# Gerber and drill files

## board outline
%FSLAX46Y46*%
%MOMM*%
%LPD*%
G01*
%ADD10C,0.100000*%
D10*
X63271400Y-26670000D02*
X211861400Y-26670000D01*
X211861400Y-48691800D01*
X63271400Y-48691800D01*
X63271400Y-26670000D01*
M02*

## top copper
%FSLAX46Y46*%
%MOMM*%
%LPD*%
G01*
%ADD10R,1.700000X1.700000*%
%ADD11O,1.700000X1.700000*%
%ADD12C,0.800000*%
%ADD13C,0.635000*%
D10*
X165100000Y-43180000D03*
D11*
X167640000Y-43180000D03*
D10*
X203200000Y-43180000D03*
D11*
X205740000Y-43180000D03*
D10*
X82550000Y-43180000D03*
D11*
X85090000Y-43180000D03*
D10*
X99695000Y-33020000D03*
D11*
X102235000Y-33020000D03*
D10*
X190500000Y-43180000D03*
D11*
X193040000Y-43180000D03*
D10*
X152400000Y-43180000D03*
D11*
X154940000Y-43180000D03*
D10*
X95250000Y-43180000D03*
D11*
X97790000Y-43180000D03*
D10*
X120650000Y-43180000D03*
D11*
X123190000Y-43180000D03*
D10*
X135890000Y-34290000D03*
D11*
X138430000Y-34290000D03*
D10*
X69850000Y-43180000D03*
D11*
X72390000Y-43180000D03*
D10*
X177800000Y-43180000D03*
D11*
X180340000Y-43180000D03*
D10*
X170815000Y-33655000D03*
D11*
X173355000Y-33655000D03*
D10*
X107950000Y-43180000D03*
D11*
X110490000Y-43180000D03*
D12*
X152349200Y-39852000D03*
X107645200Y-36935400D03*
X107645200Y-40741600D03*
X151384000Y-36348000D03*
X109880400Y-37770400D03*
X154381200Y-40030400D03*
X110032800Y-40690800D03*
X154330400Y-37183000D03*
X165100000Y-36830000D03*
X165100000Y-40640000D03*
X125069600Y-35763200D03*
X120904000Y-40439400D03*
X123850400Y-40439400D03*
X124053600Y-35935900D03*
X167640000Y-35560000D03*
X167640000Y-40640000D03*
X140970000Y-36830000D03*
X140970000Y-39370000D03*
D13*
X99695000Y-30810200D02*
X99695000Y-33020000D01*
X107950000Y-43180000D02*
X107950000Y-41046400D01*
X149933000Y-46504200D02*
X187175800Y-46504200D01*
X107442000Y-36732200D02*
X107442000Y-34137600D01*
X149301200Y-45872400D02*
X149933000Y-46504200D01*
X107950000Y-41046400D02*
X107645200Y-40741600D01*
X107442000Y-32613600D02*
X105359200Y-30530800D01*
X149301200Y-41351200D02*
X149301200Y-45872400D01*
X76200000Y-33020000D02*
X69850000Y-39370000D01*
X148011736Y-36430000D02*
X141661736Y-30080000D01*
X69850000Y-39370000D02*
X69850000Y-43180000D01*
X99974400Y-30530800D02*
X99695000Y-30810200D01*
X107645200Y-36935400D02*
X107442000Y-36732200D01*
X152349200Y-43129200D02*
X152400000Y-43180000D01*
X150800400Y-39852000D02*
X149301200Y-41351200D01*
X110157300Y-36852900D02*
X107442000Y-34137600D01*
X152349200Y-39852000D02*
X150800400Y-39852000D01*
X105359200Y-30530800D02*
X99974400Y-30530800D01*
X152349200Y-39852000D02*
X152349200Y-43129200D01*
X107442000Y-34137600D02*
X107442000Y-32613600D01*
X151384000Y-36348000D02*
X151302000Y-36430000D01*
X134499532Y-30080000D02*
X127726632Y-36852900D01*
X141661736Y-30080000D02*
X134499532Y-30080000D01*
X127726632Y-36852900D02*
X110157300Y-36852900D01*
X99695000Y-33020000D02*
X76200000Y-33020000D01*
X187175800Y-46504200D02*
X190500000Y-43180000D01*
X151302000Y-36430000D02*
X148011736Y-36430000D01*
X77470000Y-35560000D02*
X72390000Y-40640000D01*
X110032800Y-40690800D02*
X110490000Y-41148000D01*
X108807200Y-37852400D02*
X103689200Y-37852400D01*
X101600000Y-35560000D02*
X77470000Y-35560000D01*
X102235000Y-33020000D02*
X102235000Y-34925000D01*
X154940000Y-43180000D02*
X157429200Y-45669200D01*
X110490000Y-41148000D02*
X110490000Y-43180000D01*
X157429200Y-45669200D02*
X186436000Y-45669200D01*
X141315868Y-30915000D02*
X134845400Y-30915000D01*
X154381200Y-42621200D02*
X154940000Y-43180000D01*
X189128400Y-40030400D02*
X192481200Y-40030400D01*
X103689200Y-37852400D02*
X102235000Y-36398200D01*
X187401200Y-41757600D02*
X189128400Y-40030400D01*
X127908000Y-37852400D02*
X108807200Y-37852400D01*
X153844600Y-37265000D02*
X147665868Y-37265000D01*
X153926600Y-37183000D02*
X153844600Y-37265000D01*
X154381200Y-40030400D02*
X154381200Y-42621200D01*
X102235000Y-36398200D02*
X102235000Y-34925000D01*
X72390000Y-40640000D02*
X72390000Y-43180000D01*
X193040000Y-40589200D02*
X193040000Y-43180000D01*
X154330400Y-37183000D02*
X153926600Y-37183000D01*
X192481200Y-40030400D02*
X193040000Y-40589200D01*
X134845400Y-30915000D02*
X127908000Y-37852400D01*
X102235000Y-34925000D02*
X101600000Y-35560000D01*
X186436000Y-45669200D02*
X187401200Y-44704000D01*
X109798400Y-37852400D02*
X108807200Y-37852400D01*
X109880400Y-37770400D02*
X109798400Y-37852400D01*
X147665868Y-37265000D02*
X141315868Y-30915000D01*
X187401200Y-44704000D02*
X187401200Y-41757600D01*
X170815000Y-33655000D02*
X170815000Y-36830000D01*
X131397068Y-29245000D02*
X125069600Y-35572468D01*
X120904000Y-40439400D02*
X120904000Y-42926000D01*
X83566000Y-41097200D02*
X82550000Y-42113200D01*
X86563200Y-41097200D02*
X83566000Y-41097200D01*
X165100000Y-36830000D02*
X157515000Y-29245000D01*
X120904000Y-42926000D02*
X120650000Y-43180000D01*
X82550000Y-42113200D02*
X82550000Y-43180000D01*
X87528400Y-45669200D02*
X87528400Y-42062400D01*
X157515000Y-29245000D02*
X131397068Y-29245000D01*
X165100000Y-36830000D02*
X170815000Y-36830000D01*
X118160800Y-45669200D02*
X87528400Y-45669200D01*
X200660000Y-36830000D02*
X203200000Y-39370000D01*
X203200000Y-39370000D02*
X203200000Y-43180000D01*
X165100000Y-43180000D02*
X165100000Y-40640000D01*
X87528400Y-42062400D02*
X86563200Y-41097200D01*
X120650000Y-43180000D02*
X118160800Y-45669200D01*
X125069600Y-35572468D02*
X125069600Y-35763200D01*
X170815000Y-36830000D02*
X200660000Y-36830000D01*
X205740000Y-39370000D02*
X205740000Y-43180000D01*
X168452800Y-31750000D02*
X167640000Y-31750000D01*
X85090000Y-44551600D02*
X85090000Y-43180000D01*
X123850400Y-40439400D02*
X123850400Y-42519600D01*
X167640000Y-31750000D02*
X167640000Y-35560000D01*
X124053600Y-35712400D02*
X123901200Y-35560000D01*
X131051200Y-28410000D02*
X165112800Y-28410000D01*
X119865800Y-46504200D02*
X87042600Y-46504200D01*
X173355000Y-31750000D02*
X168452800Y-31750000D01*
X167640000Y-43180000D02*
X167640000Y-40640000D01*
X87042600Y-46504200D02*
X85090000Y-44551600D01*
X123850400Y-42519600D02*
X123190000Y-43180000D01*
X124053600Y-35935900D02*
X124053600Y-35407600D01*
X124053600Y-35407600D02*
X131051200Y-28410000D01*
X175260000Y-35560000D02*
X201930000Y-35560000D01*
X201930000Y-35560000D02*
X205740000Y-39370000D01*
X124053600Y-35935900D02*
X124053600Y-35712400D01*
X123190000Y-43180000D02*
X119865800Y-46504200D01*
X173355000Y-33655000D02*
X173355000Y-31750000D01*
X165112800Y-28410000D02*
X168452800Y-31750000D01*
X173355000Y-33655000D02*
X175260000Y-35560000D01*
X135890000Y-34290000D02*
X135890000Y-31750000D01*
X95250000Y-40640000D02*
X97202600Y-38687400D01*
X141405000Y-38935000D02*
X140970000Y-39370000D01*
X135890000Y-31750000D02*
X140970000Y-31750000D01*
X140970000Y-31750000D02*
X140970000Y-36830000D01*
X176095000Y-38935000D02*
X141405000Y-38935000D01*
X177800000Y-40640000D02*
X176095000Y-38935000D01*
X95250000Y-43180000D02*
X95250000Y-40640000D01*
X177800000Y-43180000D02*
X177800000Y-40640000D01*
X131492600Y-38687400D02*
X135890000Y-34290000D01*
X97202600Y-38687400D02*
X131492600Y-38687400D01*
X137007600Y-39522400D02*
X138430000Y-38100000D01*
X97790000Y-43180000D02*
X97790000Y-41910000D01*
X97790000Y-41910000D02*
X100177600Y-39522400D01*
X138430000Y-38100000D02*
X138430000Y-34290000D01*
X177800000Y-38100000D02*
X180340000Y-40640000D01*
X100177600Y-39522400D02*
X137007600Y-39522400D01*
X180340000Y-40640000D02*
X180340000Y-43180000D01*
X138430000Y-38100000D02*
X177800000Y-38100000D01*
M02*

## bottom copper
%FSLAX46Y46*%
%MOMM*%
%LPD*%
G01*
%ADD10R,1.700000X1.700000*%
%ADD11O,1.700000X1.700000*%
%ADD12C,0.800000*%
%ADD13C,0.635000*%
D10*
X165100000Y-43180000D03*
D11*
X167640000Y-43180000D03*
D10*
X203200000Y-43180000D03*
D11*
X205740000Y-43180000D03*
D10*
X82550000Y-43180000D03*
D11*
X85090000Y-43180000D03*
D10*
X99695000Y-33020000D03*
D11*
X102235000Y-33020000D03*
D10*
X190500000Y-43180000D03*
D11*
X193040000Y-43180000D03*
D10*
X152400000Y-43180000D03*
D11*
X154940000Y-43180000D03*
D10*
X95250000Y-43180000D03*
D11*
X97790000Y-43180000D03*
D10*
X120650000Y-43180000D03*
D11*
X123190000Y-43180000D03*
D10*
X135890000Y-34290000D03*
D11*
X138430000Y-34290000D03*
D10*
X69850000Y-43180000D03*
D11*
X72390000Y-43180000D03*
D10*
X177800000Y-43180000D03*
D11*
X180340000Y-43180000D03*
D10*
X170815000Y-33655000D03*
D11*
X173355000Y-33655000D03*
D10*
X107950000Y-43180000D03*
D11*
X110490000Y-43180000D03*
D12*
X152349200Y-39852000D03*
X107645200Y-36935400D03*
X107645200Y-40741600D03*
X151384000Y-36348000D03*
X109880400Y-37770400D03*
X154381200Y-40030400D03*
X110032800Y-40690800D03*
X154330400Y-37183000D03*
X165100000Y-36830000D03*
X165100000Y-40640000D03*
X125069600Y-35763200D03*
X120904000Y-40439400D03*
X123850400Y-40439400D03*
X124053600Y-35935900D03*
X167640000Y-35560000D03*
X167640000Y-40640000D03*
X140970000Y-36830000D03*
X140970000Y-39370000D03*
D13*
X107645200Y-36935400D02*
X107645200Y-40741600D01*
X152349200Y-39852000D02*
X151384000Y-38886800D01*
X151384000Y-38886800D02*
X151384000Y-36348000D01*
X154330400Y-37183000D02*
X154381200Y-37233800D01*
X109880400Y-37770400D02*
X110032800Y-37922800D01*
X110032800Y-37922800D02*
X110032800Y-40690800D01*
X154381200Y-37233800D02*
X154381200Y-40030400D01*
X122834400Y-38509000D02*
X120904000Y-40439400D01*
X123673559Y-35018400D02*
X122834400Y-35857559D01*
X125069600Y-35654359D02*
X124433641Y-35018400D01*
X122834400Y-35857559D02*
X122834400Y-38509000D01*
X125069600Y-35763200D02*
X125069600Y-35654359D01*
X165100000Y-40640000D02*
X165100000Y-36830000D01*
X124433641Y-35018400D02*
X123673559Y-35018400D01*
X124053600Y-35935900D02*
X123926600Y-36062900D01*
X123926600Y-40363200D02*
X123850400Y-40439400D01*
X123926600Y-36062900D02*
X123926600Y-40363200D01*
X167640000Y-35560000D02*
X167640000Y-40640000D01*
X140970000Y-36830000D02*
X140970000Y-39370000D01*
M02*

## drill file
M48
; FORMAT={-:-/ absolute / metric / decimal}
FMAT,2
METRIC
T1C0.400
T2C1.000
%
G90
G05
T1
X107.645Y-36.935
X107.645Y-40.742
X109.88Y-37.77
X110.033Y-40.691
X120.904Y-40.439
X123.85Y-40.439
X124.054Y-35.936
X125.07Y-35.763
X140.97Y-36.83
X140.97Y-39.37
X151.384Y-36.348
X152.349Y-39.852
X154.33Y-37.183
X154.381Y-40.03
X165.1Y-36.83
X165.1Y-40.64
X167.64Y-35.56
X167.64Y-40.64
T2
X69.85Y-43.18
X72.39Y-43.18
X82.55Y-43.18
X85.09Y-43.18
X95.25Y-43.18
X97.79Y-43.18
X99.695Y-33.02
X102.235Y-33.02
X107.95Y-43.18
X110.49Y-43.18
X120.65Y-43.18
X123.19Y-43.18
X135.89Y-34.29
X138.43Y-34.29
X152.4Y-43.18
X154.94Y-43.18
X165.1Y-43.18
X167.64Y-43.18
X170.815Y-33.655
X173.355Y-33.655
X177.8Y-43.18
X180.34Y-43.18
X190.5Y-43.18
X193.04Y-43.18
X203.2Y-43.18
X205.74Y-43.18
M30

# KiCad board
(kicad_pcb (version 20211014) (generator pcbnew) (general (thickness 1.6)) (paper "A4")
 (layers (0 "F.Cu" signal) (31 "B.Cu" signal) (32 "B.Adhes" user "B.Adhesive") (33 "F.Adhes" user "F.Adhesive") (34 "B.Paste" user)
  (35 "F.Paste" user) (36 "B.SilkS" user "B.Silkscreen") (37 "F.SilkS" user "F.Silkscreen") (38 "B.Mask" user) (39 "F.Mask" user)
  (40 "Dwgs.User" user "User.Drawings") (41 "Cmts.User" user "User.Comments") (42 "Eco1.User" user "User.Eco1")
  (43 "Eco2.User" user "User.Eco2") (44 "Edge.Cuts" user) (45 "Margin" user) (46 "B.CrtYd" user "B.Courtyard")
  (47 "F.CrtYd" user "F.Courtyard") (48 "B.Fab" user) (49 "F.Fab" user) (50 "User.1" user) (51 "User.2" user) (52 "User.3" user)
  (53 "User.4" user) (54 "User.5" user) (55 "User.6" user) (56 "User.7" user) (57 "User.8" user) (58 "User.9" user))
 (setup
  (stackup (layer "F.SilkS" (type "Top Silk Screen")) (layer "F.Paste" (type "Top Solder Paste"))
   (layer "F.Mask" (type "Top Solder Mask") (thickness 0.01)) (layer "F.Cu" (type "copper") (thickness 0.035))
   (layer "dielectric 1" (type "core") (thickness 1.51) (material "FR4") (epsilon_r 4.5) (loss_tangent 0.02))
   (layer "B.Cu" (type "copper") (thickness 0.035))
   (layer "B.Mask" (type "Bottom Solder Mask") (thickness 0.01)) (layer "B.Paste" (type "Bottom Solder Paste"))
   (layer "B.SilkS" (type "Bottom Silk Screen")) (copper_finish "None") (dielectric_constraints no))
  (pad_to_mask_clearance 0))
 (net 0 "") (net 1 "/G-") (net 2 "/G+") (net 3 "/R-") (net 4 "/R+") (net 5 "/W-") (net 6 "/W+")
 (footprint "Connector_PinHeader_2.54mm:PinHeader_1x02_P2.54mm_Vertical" (layer "F.Cu") (at 165.1 43.18 90)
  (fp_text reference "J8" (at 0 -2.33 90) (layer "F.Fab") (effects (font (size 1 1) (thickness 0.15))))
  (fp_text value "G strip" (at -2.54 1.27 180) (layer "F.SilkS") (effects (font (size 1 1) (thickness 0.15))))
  (pad "1" thru_hole rect (at 0 0 90) (size 1.7 1.7) (drill 1) (layers *.Cu *.Mask) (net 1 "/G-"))
  (pad "2" thru_hole oval (at 0 2.54 90) (size 1.7 1.7) (drill 1) (layers *.Cu *.Mask) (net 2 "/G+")))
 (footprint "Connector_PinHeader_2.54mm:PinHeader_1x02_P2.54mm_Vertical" (layer "F.Cu") (at 203.2 43.18 90)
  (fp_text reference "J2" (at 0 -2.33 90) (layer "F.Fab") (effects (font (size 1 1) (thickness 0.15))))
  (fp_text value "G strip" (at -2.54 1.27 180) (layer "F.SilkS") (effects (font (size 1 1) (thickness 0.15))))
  (pad "1" thru_hole rect (at 0 0 90) (size 1.7 1.7) (drill 1) (layers *.Cu *.Mask) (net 1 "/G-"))
  (pad "2" thru_hole oval (at 0 2.54 90) (size 1.7 1.7) (drill 1) (layers *.Cu *.Mask) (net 2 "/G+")))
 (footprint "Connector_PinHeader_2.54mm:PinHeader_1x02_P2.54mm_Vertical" (layer "F.Cu") (at 82.55 43.18 90)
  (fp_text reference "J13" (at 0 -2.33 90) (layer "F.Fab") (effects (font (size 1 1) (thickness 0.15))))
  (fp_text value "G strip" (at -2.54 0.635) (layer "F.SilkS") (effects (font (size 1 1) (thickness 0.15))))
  (pad "1" thru_hole rect (at 0 0 90) (size 1.7 1.7) (drill 1) (layers *.Cu *.Mask) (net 1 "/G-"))
  (pad "2" thru_hole oval (at 0 2.54 90) (size 1.7 1.7) (drill 1) (layers *.Cu *.Mask) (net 2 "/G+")))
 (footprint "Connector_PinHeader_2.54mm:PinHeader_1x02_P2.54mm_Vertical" (layer "F.Cu") (at 99.695 33.02 90)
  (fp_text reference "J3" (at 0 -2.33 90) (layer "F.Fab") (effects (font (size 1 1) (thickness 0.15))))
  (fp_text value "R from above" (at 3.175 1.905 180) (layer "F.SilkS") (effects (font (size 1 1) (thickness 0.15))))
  (pad "1" thru_hole rect (at 0 0 90) (size 1.7 1.7) (drill 1) (layers *.Cu *.Mask) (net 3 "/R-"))
  (pad "2" thru_hole oval (at 0 2.54 90) (size 1.7 1.7) (drill 1) (layers *.Cu *.Mask) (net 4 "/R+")))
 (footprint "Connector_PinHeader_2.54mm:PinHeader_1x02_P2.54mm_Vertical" (layer "F.Cu") (at 190.5 43.18 90)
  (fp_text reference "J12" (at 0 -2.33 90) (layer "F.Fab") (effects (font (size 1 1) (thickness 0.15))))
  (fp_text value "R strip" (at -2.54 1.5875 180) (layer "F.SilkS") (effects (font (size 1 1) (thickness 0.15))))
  (pad "1" thru_hole rect (at 0 0 90) (size 1.7 1.7) (drill 1) (layers *.Cu *.Mask) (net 3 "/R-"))
  (pad "2" thru_hole oval (at 0 2.54 90) (size 1.7 1.7) (drill 1) (layers *.Cu *.Mask) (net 4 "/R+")))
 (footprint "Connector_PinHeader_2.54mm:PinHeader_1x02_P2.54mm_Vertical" (layer "F.Cu") (at 152.4 43.18 90)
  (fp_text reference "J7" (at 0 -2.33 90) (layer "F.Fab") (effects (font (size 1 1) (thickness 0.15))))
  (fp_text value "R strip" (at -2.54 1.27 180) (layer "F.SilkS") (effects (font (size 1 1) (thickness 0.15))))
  (pad "1" thru_hole rect (at 0 0 90) (size 1.7 1.7) (drill 1) (layers *.Cu *.Mask) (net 3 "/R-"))
  (pad "2" thru_hole oval (at 0 2.54 90) (size 1.7 1.7) (drill 1) (layers *.Cu *.Mask) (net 4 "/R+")))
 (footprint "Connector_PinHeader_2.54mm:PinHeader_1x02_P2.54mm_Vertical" (layer "F.Cu") (at 95.25 43.18 90)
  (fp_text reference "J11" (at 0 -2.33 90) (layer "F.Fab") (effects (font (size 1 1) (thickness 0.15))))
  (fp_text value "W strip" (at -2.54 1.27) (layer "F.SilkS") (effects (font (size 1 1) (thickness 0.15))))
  (pad "1" thru_hole rect (at 0 0 90) (size 1.7 1.7) (drill 1) (layers *.Cu *.Mask) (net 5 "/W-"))
  (pad "2" thru_hole oval (at 0 2.54 90) (size 1.7 1.7) (drill 1) (layers *.Cu *.Mask) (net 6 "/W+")))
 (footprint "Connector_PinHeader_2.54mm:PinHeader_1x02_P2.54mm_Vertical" (layer "F.Cu") (at 120.65 43.18 90)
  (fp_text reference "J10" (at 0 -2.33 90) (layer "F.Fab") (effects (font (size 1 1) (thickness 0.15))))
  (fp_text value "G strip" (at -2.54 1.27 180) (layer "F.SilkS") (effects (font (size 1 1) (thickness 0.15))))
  (pad "1" thru_hole rect (at 0 0 90) (size 1.7 1.7) (drill 1) (layers *.Cu *.Mask) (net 1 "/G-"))
  (pad "2" thru_hole oval (at 0 2.54 90) (size 1.7 1.7) (drill 1) (layers *.Cu *.Mask) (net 2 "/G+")))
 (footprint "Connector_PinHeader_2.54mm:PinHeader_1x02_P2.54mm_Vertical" (layer "F.Cu") (at 135.89 34.29 90)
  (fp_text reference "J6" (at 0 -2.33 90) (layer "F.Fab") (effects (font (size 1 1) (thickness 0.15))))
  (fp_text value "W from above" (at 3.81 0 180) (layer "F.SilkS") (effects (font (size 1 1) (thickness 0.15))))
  (pad "1" thru_hole rect (at 0 0 90) (size 1.7 1.7) (drill 1) (layers *.Cu *.Mask) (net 5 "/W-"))
  (pad "2" thru_hole oval (at 0 2.54 90) (size 1.7 1.7) (drill 1) (layers *.Cu *.Mask) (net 6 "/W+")))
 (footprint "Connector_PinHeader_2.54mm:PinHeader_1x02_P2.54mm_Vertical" (layer "F.Cu") (at 69.85 43.18 90)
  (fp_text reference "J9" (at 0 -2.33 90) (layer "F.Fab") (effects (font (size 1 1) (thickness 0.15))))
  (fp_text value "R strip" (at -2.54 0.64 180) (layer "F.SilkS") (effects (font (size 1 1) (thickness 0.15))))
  (pad "1" thru_hole rect (at 0 0 90) (size 1.7 1.7) (drill 1) (layers *.Cu *.Mask) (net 3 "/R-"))
  (pad "2" thru_hole oval (at 0 2.54 90) (size 1.7 1.7) (drill 1) (layers *.Cu *.Mask) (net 4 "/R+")))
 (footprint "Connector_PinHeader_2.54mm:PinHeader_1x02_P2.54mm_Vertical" (layer "F.Cu") (at 177.8 43.18 90)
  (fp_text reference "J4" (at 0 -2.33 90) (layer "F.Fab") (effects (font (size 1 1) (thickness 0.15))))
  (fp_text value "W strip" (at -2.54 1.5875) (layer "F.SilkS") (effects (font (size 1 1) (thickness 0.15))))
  (pad "1" thru_hole rect (at 0 0 90) (size 1.7 1.7) (drill 1) (layers *.Cu *.Mask) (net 5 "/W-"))
  (pad "2" thru_hole oval (at 0 2.54 90) (size 1.7 1.7) (drill 1) (layers *.Cu *.Mask) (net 6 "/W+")))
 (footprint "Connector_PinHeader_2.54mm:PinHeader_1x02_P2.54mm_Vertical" (layer "F.Cu") (at 170.815 33.655 90)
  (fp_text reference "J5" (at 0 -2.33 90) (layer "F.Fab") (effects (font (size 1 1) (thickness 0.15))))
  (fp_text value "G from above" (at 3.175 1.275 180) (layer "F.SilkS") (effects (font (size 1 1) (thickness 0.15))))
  (pad "1" thru_hole rect (at 0 0 90) (size 1.7 1.7) (drill 1) (layers *.Cu *.Mask) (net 1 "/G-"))
  (pad "2" thru_hole oval (at 0 2.54 90) (size 1.7 1.7) (drill 1) (layers *.Cu *.Mask) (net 2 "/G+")))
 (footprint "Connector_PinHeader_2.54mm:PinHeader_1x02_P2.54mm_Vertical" (layer "F.Cu") (at 107.95 43.18 90)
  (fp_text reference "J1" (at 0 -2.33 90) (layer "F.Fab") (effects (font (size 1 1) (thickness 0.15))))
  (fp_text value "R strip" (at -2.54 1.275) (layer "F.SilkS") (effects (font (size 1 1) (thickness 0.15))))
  (pad "1" thru_hole rect (at 0 0 90) (size 1.7 1.7) (drill 1) (layers *.Cu *.Mask) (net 3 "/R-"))
  (pad "2" thru_hole oval (at 0 2.54 90) (size 1.7 1.7) (drill 1) (layers *.Cu *.Mask) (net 4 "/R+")))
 (gr_rect (start 63.2714 26.67) (end 211.8614 48.6918) (layer "Edge.Cuts") (width 0.1) (fill none))
 (segment (start 99.695 30.8102) (end 99.695 33.02) (width 0.635) (layer "F.Cu") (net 3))
 (segment (start 107.95 43.18) (end 107.95 41.0464) (width 0.635) (layer "F.Cu") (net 3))
 (segment (start 149.933 46.5042) (end 187.1758 46.5042) (width 0.635) (layer "F.Cu") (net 3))
 (segment (start 107.442 36.7322) (end 107.442 34.1376) (width 0.635) (layer "F.Cu") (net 3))
 (segment (start 149.3012 45.8724) (end 149.933 46.5042) (width 0.635) (layer "F.Cu") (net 3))
 (segment (start 107.95 41.0464) (end 107.6452 40.7416) (width 0.635) (layer "F.Cu") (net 3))
 (segment (start 107.442 32.6136) (end 105.3592 30.5308) (width 0.635) (layer "F.Cu") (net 3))
 (segment (start 149.3012 41.3512) (end 149.3012 45.8724) (width 0.635) (layer "F.Cu") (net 3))
 (segment (start 76.2 33.02) (end 69.85 39.37) (width 0.635) (layer "F.Cu") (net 3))
 (segment (start 148.011736 36.43) (end 141.661736 30.08) (width 0.635) (layer "F.Cu") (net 3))
 (segment (start 69.85 39.37) (end 69.85 43.18) (width 0.635) (layer "F.Cu") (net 3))
 (segment (start 99.9744 30.5308) (end 99.695 30.8102) (width 0.635) (layer "F.Cu") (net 3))
 (segment (start 107.6452 36.9354) (end 107.442 36.7322) (width 0.635) (layer "F.Cu") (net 3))
 (segment (start 152.3492 43.1292) (end 152.4 43.18) (width 0.635) (layer "F.Cu") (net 3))
 (segment (start 150.8004 39.852) (end 149.3012 41.3512) (width 0.635) (layer "F.Cu") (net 3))
 (segment (start 110.1573 36.8529) (end 107.442 34.1376) (width 0.635) (layer "F.Cu") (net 3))
 (segment (start 152.3492 39.852) (end 150.8004 39.852) (width 0.635) (layer "F.Cu") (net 3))
 (segment (start 105.3592 30.5308) (end 99.9744 30.5308) (width 0.635) (layer "F.Cu") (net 3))
 (segment (start 152.3492 39.852) (end 152.3492 43.1292) (width 0.635) (layer "F.Cu") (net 3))
 (segment (start 107.442 34.1376) (end 107.442 32.6136) (width 0.635) (layer "F.Cu") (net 3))
 (segment (start 151.384 36.348) (end 151.302 36.43) (width 0.635) (layer "F.Cu") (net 3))
 (segment (start 134.499532 30.08) (end 127.726632 36.8529) (width 0.635) (layer "F.Cu") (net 3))
 (segment (start 141.661736 30.08) (end 134.499532 30.08) (width 0.635) (layer "F.Cu") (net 3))
 (segment (start 127.726632 36.8529) (end 110.1573 36.8529) (width 0.635) (layer "F.Cu") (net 3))
 (segment (start 99.695 33.02) (end 76.2 33.02) (width 0.635) (layer "F.Cu") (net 3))
 (segment (start 187.1758 46.5042) (end 190.5 43.18) (width 0.635) (layer "F.Cu") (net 3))
 (segment (start 151.302 36.43) (end 148.011736 36.43) (width 0.635) (layer "F.Cu") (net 3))
 (via (at 152.3492 39.852) (size 0.8) (drill 0.4) (layers "F.Cu" "B.Cu") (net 3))
 (via (at 107.6452 36.9354) (size 0.8) (drill 0.4) (layers "F.Cu" "B.Cu") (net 3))
 (via (at 107.6452 40.7416) (size 0.8) (drill 0.4) (layers "F.Cu" "B.Cu") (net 3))
 (via (at 151.384 36.348) (size 0.8) (drill 0.4) (layers "F.Cu" "B.Cu") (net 3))
 (segment (start 107.6452 36.9354) (end 107.6452 40.7416) (width 0.635) (layer "B.Cu") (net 3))
 (segment (start 152.3492 39.852) (end 151.384 38.8868) (width 0.635) (layer "B.Cu") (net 3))
 (segment (start 151.384 38.8868) (end 151.384 36.348) (width 0.635) (layer "B.Cu") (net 3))
 (segment (start 77.47 35.56) (end 72.39 40.64) (width 0.635) (layer "F.Cu") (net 4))
 (segment (start 110.0328 40.6908) (end 110.49 41.148) (width 0.635) (layer "F.Cu") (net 4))
 (segment (start 108.8072 37.8524) (end 103.6892 37.8524) (width 0.635) (layer "F.Cu") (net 4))
 (segment (start 101.6 35.56) (end 77.47 35.56) (width 0.635) (layer "F.Cu") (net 4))
 (segment (start 102.235 33.02) (end 102.235 34.925) (width 0.635) (layer "F.Cu") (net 4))
 (segment (start 154.94 43.18) (end 157.4292 45.6692) (width 0.635) (layer "F.Cu") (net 4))
 (segment (start 110.49 41.148) (end 110.49 43.18) (width 0.635) (layer "F.Cu") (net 4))
 (segment (start 157.4292 45.6692) (end 186.436 45.6692) (width 0.635) (layer "F.Cu") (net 4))
 (segment (start 141.315868 30.915) (end 134.8454 30.915) (width 0.635) (layer "F.Cu") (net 4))
 (segment (start 154.3812 42.6212) (end 154.94 43.18) (width 0.635) (layer "F.Cu") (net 4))
 (segment (start 189.1284 40.0304) (end 192.4812 40.0304) (width 0.635) (layer "F.Cu") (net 4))
 (segment (start 103.6892 37.8524) (end 102.235 36.3982) (width 0.635) (layer "F.Cu") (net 4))
 (segment (start 187.4012 41.7576) (end 189.1284 40.0304) (width 0.635) (layer "F.Cu") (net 4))
 (segment (start 127.908 37.8524) (end 108.8072 37.8524) (width 0.635) (layer "F.Cu") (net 4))
 (segment (start 153.8446 37.265) (end 147.665868 37.265) (width 0.635) (layer "F.Cu") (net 4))
 (segment (start 153.9266 37.183) (end 153.8446 37.265) (width 0.635) (layer "F.Cu") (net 4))
 (segment (start 154.3812 40.0304) (end 154.3812 42.6212) (width 0.635) (layer "F.Cu") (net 4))
 (segment (start 102.235 36.3982) (end 102.235 34.925) (width 0.635) (layer "F.Cu") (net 4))
 (segment (start 72.39 40.64) (end 72.39 43.18) (width 0.635) (layer "F.Cu") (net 4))
 (segment (start 193.04 40.5892) (end 193.04 43.18) (width 0.635) (layer "F.Cu") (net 4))
 (segment (start 154.3304 37.183) (end 153.9266 37.183) (width 0.635) (layer "F.Cu") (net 4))
 (segment (start 192.4812 40.0304) (end 193.04 40.5892) (width 0.635) (layer "F.Cu") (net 4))
 (segment (start 134.8454 30.915) (end 127.908 37.8524) (width 0.635) (layer "F.Cu") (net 4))
 (segment (start 102.235 34.925) (end 101.6 35.56) (width 0.635) (layer "F.Cu") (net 4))
 (segment (start 186.436 45.6692) (end 187.4012 44.704) (width 0.635) (layer "F.Cu") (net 4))
 (segment (start 109.7984 37.8524) (end 108.8072 37.8524) (width 0.635) (layer "F.Cu") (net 4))
 (segment (start 109.8804 37.7704) (end 109.7984 37.8524) (width 0.635) (layer "F.Cu") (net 4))
 (segment (start 147.665868 37.265) (end 141.315868 30.915) (width 0.635) (layer "F.Cu") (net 4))
 (segment (start 187.4012 44.704) (end 187.4012 41.7576) (width 0.635) (layer "F.Cu") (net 4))
 (via (at 109.8804 37.7704) (size 0.8) (drill 0.4) (layers "F.Cu" "B.Cu") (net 4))
 (via (at 154.3812 40.0304) (size 0.8) (drill 0.4) (layers "F.Cu" "B.Cu") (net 4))
 (via (at 110.0328 40.6908) (size 0.8) (drill 0.4) (layers "F.Cu" "B.Cu") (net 4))
 (via (at 154.3304 37.183) (size 0.8) (drill 0.4) (layers "F.Cu" "B.Cu") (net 4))
 (segment (start 154.3304 37.183) (end 154.3812 37.2338) (width 0.635) (layer "B.Cu") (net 4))
 (segment (start 109.8804 37.7704) (end 110.0328 37.9228) (width 0.635) (layer "B.Cu") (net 4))
 (segment (start 110.0328 37.9228) (end 110.0328 40.6908) (width 0.635) (layer "B.Cu") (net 4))
 (segment (start 154.3812 37.2338) (end 154.3812 40.0304) (width 0.635) (layer "B.Cu") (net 4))
 (segment (start 170.815 33.655) (end 170.815 36.83) (width 0.635) (layer "F.Cu") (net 1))
 (segment (start 131.397068 29.245) (end 125.0696 35.572468) (width 0.635) (layer "F.Cu") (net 1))
 (segment (start 120.904 40.4394) (end 120.904 42.926) (width 0.635) (layer "F.Cu") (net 1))
 (segment (start 83.566 41.0972) (end 82.55 42.1132) (width 0.635) (layer "F.Cu") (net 1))
 (segment (start 86.5632 41.0972) (end 83.566 41.0972) (width 0.635) (layer "F.Cu") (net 1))
 (segment (start 165.1 36.83) (end 157.515 29.245) (width 0.635) (layer "F.Cu") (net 1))
 (segment (start 120.904 42.926) (end 120.65 43.18) (width 0.635) (layer "F.Cu") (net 1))
 (segment (start 82.55 42.1132) (end 82.55 43.18) (width 0.635) (layer "F.Cu") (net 1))
 (segment (start 87.5284 45.6692) (end 87.5284 42.0624) (width 0.635) (layer "F.Cu") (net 1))
 (segment (start 157.515 29.245) (end 131.397068 29.245) (width 0.635) (layer "F.Cu") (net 1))
 (segment (start 165.1 36.83) (end 170.815 36.83) (width 0.635) (layer "F.Cu") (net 1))
 (segment (start 118.1608 45.6692) (end 87.5284 45.6692) (width 0.635) (layer "F.Cu") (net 1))
 (segment (start 200.66 36.83) (end 203.2 39.37) (width 0.635) (layer "F.Cu") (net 1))
 (segment (start 203.2 39.37) (end 203.2 43.18) (width 0.635) (layer "F.Cu") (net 1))
 (segment (start 165.1 43.18) (end 165.1 40.64) (width 0.635) (layer "F.Cu") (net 1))
 (segment (start 87.5284 42.0624) (end 86.5632 41.0972) (width 0.635) (layer "F.Cu") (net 1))
 (segment (start 120.65 43.18) (end 118.1608 45.6692) (width 0.635) (layer "F.Cu") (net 1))
 (segment (start 125.0696 35.572468) (end 125.0696 35.7632) (width 0.635) (layer "F.Cu") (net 1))
 (segment (start 170.815 36.83) (end 200.66 36.83) (width 0.635) (layer "F.Cu") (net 1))
 (via (at 165.1 36.83) (size 0.8) (drill 0.4) (layers "F.Cu" "B.Cu") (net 1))
 (via (at 165.1 40.64) (size 0.8) (drill 0.4) (layers "F.Cu" "B.Cu") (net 1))
 (via (at 125.0696 35.7632) (size 0.8) (drill 0.4) (layers "F.Cu" "B.Cu") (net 1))
 (via (at 120.904 40.4394) (size 0.8) (drill 0.4) (layers "F.Cu" "B.Cu") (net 1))
 (segment (start 122.8344 38.509) (end 120.904 40.4394) (width 0.635) (layer "B.Cu") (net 1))
 (segment (start 123.673559 35.0184) (end 122.8344 35.857559) (width 0.635) (layer "B.Cu") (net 1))
 (segment (start 125.0696 35.654359) (end 124.433641 35.0184) (width 0.635) (layer "B.Cu") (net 1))
 (segment (start 122.8344 35.857559) (end 122.8344 38.509) (width 0.635) (layer "B.Cu") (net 1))
 (segment (start 125.0696 35.7632) (end 125.0696 35.654359) (width 0.635) (layer "B.Cu") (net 1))
 (segment (start 165.1 40.64) (end 165.1 36.83) (width 0.635) (layer "B.Cu") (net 1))
 (segment (start 124.433641 35.0184) (end 123.673559 35.0184) (width 0.635) (layer "B.Cu") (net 1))
 (segment (start 205.74 39.37) (end 205.74 43.18) (width 0.635) (layer "F.Cu") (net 2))
 (segment (start 168.4528 31.75) (end 167.64 31.75) (width 0.635) (layer "F.Cu") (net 2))
 (segment (start 85.09 44.5516) (end 85.09 43.18) (width 0.635) (layer "F.Cu") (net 2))
 (segment (start 123.8504 40.4394) (end 123.8504 42.5196) (width 0.635) (layer "F.Cu") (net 2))
 (segment (start 167.64 31.75) (end 167.64 35.56) (width 0.635) (layer "F.Cu") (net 2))
 (segment (start 124.0536 35.7124) (end 123.9012 35.56) (width 0.635) (layer "F.Cu") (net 2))
 (segment (start 131.0512 28.41) (end 165.1128 28.41) (width 0.635) (layer "F.Cu") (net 2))
 (segment (start 119.8658 46.5042) (end 87.0426 46.5042) (width 0.635) (layer "F.Cu") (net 2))
 (segment (start 173.355 31.75) (end 168.4528 31.75) (width 0.635) (layer "F.Cu") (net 2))
 (segment (start 167.64 43.18) (end 167.64 40.64) (width 0.635) (layer "F.Cu") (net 2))
 (segment (start 87.0426 46.5042) (end 85.09 44.5516) (width 0.635) (layer "F.Cu") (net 2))
 (segment (start 123.8504 42.5196) (end 123.19 43.18) (width 0.635) (layer "F.Cu") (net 2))
 (segment (start 124.0536 35.9359) (end 124.0536 35.4076) (width 0.635) (layer "F.Cu") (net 2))
 (segment (start 124.0536 35.4076) (end 131.0512 28.41) (width 0.635) (layer "F.Cu") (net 2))
 (segment (start 175.26 35.56) (end 201.93 35.56) (width 0.635) (layer "F.Cu") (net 2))
 (segment (start 201.93 35.56) (end 205.74 39.37) (width 0.635) (layer "F.Cu") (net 2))
 (segment (start 124.0536 35.9359) (end 124.0536 35.7124) (width 0.635) (layer "F.Cu") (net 2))
 (segment (start 123.19 43.18) (end 119.8658 46.5042) (width 0.635) (layer "F.Cu") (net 2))
 (segment (start 173.355 33.655) (end 173.355 31.75) (width 0.635) (layer "F.Cu") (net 2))
 (segment (start 165.1128 28.41) (end 168.4528 31.75) (width 0.635) (layer "F.Cu") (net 2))
 (segment (start 173.355 33.655) (end 175.26 35.56) (width 0.635) (layer "F.Cu") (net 2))
 (via (at 123.8504 40.4394) (size 0.8) (drill 0.4) (layers "F.Cu" "B.Cu") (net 2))
 (via (at 124.0536 35.9359) (size 0.8) (drill 0.4) (layers "F.Cu" "B.Cu") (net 2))
 (via (at 167.64 35.56) (size 0.8) (drill 0.4) (layers "F.Cu" "B.Cu") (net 2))
 (via (at 167.64 40.64) (size 0.8) (drill 0.4) (layers "F.Cu" "B.Cu") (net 2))
 (segment (start 124.0536 35.9359) (end 123.9266 36.0629) (width 0.635) (layer "B.Cu") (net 2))
 (segment (start 123.9266 40.3632) (end 123.8504 40.4394) (width 0.635) (layer "B.Cu") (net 2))
 (segment (start 123.9266 36.0629) (end 123.9266 40.3632) (width 0.635) (layer "B.Cu") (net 2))
 (segment (start 167.64 35.56) (end 167.64 40.64) (width 0.635) (layer "B.Cu") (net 2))
 (segment (start 135.89 34.29) (end 135.89 31.75) (width 0.635) (layer "F.Cu") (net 5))
 (segment (start 95.25 40.64) (end 97.2026 38.6874) (width 0.635) (layer "F.Cu") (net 5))
 (segment (start 141.405 38.935) (end 140.97 39.37) (width 0.635) (layer "F.Cu") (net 5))
 (segment (start 135.89 31.75) (end 140.97 31.75) (width 0.635) (layer "F.Cu") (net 5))
 (segment (start 140.97 31.75) (end 140.97 36.83) (width 0.635) (layer "F.Cu") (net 5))
 (segment (start 176.095 38.935) (end 141.405 38.935) (width 0.635) (layer "F.Cu") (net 5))
 (segment (start 177.8 40.64) (end 176.095 38.935) (width 0.635) (layer "F.Cu") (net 5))
 (segment (start 95.25 43.18) (end 95.25 40.64) (width 0.635) (layer "F.Cu") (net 5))
 (segment (start 177.8 43.18) (end 177.8 40.64) (width 0.635) (layer "F.Cu") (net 5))
 (segment (start 131.4926 38.6874) (end 135.89 34.29) (width 0.635) (layer "F.Cu") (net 5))
 (segment (start 97.2026 38.6874) (end 131.4926 38.6874) (width 0.635) (layer "F.Cu") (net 5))
 (via (at 140.97 36.83) (size 0.8) (drill 0.4) (layers "F.Cu" "B.Cu") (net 5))
 (via (at 140.97 39.37) (size 0.8) (drill 0.4) (layers "F.Cu" "B.Cu") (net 5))
 (segment (start 140.97 36.83) (end 140.97 39.37) (width 0.635) (layer "B.Cu") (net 5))
 (segment (start 137.0076 39.5224) (end 138.43 38.1) (width 0.635) (layer "F.Cu") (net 6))
 (segment (start 97.79 43.18) (end 97.79 41.91) (width 0.635) (layer "F.Cu") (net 6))
 (segment (start 97.79 41.91) (end 100.1776 39.5224) (width 0.635) (layer "F.Cu") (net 6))
 (segment (start 138.43 38.1) (end 138.43 34.29) (width 0.635) (layer "F.Cu") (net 6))
 (segment (start 177.8 38.1) (end 180.34 40.64) (width 0.635) (layer "F.Cu") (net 6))
 (segment (start 100.1776 39.5224) (end 137.0076 39.5224) (width 0.635) (layer "F.Cu") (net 6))
 (segment (start 180.34 40.64) (end 180.34 43.18) (width 0.635) (layer "F.Cu") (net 6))
 (segment (start 138.43 38.1) (end 177.8 38.1) (width 0.635) (layer "F.Cu") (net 6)))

